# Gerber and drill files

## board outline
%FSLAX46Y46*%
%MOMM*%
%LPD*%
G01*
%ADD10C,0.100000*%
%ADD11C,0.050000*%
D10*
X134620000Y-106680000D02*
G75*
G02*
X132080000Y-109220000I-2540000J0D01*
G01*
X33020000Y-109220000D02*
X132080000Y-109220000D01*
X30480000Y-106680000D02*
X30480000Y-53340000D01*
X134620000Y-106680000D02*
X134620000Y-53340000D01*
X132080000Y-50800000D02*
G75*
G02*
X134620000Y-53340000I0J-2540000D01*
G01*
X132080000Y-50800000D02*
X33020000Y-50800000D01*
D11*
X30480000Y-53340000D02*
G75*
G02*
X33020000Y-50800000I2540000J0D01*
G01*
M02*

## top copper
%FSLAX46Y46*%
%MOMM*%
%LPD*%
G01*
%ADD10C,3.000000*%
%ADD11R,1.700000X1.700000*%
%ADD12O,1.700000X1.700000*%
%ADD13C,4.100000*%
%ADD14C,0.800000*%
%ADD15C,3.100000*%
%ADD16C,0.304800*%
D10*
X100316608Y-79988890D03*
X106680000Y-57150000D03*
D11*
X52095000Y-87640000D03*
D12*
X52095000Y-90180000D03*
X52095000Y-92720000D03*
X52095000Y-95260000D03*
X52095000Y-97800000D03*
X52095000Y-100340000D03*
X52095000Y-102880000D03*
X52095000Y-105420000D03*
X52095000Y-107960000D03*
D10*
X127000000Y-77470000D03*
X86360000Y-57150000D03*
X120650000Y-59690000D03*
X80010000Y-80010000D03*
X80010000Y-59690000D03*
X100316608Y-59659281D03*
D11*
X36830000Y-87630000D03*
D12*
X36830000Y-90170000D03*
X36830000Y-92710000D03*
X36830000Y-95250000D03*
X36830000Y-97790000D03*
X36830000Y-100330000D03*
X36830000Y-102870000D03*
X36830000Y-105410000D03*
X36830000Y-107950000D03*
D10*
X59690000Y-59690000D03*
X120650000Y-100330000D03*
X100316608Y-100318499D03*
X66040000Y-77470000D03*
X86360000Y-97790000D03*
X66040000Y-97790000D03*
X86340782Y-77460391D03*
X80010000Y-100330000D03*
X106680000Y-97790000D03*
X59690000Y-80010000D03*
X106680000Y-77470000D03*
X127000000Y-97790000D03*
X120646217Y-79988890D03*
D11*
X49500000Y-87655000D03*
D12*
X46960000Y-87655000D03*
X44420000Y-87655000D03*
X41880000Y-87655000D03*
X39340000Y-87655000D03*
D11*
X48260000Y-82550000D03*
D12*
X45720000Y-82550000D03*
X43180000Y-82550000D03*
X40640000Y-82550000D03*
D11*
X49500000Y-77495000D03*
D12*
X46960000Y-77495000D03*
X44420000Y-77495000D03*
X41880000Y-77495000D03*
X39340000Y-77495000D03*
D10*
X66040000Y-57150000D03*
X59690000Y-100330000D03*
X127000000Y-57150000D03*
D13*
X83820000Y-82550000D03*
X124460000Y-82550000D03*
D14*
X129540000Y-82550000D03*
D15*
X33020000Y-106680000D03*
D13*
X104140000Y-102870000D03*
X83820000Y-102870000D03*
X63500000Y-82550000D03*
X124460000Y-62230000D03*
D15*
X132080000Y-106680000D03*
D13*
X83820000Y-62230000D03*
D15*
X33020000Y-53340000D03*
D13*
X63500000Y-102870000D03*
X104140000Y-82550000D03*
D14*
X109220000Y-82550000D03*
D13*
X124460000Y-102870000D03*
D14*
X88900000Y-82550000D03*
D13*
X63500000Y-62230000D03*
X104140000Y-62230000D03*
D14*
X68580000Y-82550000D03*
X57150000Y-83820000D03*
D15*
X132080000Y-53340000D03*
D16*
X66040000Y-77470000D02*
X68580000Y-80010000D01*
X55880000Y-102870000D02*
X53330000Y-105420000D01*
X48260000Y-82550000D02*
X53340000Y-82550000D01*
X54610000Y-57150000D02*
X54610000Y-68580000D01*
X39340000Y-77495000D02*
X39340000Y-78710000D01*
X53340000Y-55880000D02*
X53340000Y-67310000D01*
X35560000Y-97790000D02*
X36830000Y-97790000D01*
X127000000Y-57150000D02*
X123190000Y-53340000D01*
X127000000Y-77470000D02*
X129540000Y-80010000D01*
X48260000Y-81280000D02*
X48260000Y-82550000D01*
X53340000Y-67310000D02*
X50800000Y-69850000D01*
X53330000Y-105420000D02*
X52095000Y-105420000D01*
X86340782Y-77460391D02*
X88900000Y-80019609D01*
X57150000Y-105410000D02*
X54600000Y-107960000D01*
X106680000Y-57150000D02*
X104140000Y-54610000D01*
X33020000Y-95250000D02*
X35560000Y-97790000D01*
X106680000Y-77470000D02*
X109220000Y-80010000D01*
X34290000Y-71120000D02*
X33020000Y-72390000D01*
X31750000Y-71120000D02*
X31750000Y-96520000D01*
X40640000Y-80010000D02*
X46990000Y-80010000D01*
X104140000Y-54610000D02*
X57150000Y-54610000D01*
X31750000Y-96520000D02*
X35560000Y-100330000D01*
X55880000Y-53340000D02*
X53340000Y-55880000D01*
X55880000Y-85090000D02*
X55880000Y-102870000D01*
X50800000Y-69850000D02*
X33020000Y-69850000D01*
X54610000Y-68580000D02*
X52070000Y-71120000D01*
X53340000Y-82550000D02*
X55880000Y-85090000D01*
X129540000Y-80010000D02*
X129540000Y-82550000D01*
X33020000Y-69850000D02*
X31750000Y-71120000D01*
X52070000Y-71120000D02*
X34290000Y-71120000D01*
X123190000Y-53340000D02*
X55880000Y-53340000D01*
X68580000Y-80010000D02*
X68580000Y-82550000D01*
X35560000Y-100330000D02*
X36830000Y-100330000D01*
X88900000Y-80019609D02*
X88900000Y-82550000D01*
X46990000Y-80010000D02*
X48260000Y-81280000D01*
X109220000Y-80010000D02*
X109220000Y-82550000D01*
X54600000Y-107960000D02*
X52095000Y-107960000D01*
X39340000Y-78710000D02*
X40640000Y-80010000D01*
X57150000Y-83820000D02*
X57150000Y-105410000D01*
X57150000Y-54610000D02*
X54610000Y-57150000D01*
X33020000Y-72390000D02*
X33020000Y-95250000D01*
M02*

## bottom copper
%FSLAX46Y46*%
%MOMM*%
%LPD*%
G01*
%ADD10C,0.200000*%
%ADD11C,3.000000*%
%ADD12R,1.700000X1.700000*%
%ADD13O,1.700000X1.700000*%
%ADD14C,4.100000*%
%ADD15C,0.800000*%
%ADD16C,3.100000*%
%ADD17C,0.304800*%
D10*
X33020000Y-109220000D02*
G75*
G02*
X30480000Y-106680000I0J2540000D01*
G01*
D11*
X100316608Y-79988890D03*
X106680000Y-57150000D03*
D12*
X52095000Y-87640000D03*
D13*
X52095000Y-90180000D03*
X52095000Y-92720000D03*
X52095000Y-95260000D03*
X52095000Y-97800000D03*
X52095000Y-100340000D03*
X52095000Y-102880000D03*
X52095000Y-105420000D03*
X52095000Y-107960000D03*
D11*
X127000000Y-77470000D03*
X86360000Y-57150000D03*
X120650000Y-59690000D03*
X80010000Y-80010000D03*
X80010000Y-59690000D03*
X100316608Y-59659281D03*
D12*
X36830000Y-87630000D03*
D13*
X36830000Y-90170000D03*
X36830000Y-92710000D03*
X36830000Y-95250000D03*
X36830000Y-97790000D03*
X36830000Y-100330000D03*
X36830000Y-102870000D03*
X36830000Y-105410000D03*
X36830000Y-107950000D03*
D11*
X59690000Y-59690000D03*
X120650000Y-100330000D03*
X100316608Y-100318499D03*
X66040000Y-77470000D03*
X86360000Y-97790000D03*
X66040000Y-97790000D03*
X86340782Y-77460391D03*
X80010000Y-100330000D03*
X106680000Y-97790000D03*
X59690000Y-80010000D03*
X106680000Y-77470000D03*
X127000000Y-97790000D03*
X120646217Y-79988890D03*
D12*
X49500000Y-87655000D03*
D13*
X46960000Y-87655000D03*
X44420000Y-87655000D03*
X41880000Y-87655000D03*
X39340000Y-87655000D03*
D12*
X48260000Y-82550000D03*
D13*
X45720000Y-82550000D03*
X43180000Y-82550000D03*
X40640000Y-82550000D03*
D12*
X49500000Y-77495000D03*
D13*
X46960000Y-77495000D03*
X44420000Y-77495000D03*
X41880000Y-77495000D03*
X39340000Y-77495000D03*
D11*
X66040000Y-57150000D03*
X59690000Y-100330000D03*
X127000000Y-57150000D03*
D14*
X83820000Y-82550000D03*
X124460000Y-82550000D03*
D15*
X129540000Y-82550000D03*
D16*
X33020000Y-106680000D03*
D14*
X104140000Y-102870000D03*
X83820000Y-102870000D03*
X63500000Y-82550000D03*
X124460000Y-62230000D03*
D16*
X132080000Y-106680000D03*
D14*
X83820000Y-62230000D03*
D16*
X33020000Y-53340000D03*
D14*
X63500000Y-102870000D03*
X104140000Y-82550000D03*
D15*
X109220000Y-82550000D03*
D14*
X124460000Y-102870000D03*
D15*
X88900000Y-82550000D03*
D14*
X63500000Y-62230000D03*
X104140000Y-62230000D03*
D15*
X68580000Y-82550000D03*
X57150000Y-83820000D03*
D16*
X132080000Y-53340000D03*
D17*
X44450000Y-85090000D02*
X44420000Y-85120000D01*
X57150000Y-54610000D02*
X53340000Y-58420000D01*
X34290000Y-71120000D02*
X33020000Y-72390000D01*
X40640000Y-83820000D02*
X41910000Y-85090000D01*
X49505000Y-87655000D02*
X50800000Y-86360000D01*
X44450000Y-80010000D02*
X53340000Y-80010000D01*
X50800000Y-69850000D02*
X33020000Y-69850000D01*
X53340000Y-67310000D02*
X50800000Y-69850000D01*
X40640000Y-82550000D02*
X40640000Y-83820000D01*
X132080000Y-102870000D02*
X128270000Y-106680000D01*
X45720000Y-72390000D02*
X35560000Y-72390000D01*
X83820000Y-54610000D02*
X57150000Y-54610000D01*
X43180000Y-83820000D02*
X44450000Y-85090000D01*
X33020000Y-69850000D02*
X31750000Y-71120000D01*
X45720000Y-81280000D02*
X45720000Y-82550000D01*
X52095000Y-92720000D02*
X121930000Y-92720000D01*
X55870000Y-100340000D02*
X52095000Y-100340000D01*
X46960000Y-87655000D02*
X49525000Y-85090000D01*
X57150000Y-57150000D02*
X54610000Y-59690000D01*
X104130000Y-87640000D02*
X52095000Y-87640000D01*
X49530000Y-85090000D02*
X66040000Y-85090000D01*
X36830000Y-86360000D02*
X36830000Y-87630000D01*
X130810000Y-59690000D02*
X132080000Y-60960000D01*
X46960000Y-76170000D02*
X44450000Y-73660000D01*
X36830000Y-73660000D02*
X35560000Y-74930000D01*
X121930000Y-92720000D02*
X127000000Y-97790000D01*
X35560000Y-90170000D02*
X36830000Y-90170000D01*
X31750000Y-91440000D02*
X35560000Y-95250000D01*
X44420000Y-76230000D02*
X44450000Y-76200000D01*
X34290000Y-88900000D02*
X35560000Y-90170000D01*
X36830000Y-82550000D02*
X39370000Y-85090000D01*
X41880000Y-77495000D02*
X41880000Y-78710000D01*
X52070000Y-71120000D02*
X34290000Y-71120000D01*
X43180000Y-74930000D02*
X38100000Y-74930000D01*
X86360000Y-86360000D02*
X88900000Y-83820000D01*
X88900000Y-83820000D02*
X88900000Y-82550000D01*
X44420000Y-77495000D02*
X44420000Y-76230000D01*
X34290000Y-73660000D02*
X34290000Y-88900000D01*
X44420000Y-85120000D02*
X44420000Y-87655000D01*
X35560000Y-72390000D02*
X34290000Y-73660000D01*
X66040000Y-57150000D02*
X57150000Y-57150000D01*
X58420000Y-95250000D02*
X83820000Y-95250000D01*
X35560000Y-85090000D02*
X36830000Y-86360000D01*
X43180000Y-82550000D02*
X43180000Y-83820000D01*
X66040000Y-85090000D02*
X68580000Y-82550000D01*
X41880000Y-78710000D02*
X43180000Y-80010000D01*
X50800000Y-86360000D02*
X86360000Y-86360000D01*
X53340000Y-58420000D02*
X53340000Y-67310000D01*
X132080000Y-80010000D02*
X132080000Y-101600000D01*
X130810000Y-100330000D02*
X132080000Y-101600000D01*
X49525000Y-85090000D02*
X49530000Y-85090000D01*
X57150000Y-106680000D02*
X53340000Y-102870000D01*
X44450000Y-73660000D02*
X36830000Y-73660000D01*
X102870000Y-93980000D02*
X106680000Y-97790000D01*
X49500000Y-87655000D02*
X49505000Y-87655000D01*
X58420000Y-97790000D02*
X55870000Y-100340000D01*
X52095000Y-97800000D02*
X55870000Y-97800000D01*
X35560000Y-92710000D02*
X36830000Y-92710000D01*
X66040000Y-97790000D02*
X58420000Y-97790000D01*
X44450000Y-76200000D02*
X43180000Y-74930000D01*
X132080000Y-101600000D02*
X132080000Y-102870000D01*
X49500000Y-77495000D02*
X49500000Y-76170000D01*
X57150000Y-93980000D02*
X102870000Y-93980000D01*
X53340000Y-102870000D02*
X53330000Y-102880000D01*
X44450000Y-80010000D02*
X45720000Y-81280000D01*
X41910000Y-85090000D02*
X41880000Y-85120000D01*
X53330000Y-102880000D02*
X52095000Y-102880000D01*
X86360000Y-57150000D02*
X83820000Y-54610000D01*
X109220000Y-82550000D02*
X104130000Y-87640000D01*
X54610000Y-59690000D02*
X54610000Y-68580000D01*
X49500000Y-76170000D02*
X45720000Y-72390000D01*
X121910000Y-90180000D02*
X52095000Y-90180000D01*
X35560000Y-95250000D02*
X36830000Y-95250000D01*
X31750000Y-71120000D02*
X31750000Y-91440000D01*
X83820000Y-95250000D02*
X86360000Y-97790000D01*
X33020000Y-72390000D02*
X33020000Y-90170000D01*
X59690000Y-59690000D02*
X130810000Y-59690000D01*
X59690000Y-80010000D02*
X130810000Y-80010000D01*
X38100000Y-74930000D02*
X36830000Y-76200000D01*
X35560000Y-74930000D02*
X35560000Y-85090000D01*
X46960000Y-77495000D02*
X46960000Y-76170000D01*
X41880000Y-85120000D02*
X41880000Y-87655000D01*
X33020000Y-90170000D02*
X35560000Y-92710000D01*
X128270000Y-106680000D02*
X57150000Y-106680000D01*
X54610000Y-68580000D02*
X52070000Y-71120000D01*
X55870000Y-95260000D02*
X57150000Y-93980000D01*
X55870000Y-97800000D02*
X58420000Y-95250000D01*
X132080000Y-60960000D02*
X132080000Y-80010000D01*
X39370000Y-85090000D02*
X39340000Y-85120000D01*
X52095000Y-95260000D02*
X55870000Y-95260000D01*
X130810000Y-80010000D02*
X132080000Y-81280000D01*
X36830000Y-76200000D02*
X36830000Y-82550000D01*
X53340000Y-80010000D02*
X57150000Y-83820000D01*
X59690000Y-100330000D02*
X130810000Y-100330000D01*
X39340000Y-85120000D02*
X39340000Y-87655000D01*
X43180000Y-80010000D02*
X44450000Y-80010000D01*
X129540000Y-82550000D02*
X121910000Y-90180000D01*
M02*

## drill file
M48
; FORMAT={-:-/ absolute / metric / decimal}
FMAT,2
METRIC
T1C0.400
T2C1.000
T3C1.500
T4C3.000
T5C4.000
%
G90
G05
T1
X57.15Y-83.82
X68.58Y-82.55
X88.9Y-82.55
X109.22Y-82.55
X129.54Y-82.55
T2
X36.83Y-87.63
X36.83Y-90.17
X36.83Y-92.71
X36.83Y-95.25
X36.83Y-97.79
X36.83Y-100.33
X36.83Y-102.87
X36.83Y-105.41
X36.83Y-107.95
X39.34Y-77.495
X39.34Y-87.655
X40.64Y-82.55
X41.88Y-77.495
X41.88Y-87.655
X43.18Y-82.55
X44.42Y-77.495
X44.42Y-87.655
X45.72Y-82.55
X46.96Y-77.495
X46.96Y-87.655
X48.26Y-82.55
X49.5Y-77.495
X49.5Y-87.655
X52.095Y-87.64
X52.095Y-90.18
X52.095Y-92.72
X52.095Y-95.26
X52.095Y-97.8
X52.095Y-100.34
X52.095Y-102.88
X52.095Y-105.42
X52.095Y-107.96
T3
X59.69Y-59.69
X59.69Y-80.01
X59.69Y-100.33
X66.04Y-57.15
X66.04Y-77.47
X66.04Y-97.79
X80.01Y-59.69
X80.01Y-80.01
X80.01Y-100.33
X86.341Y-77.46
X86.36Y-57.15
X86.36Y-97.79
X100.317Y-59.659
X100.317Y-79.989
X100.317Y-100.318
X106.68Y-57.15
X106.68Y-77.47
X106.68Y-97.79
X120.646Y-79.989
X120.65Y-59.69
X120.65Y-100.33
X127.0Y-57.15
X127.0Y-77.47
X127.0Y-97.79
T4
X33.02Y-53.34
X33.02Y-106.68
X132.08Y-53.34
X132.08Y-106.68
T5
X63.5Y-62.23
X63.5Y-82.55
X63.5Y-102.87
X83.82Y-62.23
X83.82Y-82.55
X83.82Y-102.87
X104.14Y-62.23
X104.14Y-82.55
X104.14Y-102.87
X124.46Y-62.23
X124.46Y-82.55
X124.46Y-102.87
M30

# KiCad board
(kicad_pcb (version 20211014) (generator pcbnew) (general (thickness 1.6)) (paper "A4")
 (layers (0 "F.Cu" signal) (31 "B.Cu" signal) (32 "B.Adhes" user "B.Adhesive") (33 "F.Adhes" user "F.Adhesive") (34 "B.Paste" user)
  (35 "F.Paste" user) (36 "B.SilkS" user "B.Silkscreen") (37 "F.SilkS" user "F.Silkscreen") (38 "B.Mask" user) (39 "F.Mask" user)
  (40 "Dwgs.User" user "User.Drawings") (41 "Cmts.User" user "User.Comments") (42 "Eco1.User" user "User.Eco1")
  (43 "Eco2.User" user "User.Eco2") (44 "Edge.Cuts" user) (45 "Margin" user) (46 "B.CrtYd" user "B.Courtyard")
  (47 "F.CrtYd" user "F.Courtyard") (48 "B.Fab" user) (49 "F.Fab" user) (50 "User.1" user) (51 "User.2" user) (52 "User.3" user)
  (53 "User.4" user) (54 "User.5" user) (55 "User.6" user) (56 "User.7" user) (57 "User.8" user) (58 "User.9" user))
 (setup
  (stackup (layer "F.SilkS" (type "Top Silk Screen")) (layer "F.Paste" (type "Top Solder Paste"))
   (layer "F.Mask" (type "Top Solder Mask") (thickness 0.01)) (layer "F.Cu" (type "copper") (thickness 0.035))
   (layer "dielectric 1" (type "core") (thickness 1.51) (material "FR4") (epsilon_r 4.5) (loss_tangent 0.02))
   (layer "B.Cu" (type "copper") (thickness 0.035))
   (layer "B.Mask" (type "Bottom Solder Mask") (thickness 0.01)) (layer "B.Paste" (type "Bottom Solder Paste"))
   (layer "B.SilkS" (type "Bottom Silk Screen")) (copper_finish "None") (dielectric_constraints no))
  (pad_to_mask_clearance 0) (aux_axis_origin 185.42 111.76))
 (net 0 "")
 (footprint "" (layer "F.Cu") (at 100.316608 79.98889)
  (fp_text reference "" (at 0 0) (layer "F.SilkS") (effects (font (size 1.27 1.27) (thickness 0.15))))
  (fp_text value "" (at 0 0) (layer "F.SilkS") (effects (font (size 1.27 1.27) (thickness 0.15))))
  (pad "1" thru_hole circle (at 0 0) (size 3 3) (drill 1.5) (layers *.Cu *.Mask)))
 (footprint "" (layer "F.Cu") (at 106.68 57.15)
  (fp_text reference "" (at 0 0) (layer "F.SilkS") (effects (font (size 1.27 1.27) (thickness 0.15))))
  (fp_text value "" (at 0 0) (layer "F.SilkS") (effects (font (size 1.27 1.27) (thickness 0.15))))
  (pad "1" thru_hole circle (at 0 0) (size 3 3) (drill 1.5) (layers *.Cu *.Mask)))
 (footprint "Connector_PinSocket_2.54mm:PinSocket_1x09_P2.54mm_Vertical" (layer "F.Cu") (at 52.095 87.64)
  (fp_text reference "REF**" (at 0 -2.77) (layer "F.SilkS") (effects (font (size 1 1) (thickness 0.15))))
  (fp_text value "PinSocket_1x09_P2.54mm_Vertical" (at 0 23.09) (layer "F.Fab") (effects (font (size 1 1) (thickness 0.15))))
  (pad "1" thru_hole rect (at 0 0) (size 1.7 1.7) (drill 1) (layers *.Cu *.Mask))
  (pad "2" thru_hole oval (at 0 2.54) (size 1.7 1.7) (drill 1) (layers *.Cu *.Mask))
  (pad "3" thru_hole oval (at 0 5.08) (size 1.7 1.7) (drill 1) (layers *.Cu *.Mask))
  (pad "4" thru_hole oval (at 0 7.62) (size 1.7 1.7) (drill 1) (layers *.Cu *.Mask))
  (pad "5" thru_hole oval (at 0 10.16) (size 1.7 1.7) (drill 1) (layers *.Cu *.Mask))
  (pad "6" thru_hole oval (at 0 12.7) (size 1.7 1.7) (drill 1) (layers *.Cu *.Mask))
  (pad "7" thru_hole oval (at 0 15.24) (size 1.7 1.7) (drill 1) (layers *.Cu *.Mask))
  (pad "8" thru_hole oval (at 0 17.78) (size 1.7 1.7) (drill 1) (layers *.Cu *.Mask))
  (pad "9" thru_hole oval (at 0 20.32) (size 1.7 1.7) (drill 1) (layers *.Cu *.Mask)))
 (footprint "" (layer "F.Cu") (at 127 77.47)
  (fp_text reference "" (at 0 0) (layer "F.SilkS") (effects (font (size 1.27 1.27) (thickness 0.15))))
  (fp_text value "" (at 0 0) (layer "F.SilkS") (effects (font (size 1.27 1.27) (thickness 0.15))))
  (pad "1" thru_hole circle (at 0 0) (size 3 3) (drill 1.5) (layers *.Cu *.Mask)))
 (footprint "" (layer "F.Cu") (at 86.36 57.15)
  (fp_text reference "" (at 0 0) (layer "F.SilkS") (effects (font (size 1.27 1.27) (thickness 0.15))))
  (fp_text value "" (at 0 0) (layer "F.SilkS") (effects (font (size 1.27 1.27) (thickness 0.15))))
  (pad "1" thru_hole circle (at 0 0) (size 3 3) (drill 1.5) (layers *.Cu *.Mask)))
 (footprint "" (layer "F.Cu") (at 120.65 59.69)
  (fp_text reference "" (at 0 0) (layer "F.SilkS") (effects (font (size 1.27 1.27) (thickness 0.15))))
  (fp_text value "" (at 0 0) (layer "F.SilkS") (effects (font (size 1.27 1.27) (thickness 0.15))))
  (pad "1" thru_hole circle (at 0 0) (size 3 3) (drill 1.5) (layers *.Cu *.Mask)))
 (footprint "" (layer "F.Cu") (at 80.01 80.01)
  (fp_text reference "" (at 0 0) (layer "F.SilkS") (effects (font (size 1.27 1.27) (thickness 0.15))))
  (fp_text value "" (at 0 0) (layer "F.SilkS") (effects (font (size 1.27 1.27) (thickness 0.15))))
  (pad "1" thru_hole circle (at 0 0) (size 3 3) (drill 1.5) (layers *.Cu *.Mask)))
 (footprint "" (layer "F.Cu") (at 80.01 59.69)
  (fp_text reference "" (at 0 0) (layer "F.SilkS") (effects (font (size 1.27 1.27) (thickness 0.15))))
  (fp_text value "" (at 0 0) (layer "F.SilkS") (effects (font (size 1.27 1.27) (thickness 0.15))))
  (pad "1" thru_hole circle (at 0 0) (size 3 3) (drill 1.5) (layers *.Cu *.Mask)))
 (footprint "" (layer "F.Cu") (at 100.316608 59.659281)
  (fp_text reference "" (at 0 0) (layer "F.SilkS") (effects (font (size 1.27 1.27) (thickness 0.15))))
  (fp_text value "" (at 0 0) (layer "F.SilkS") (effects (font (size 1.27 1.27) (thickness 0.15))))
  (pad "1" thru_hole circle (at 0 0) (size 3 3) (drill 1.5) (layers *.Cu *.Mask)))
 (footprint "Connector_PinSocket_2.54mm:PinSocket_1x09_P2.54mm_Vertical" (layer "F.Cu") (at 36.83 87.63)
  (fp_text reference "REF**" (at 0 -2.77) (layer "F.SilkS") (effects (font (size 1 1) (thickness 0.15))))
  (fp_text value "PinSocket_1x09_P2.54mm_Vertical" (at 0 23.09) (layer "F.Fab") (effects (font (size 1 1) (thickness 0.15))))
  (pad "1" thru_hole rect (at 0 0) (size 1.7 1.7) (drill 1) (layers *.Cu *.Mask))
  (pad "2" thru_hole oval (at 0 2.54) (size 1.7 1.7) (drill 1) (layers *.Cu *.Mask))
  (pad "3" thru_hole oval (at 0 5.08) (size 1.7 1.7) (drill 1) (layers *.Cu *.Mask))
  (pad "4" thru_hole oval (at 0 7.62) (size 1.7 1.7) (drill 1) (layers *.Cu *.Mask))
  (pad "5" thru_hole oval (at 0 10.16) (size 1.7 1.7) (drill 1) (layers *.Cu *.Mask))
  (pad "6" thru_hole oval (at 0 12.7) (size 1.7 1.7) (drill 1) (layers *.Cu *.Mask))
  (pad "7" thru_hole oval (at 0 15.24) (size 1.7 1.7) (drill 1) (layers *.Cu *.Mask))
  (pad "8" thru_hole oval (at 0 17.78) (size 1.7 1.7) (drill 1) (layers *.Cu *.Mask))
  (pad "9" thru_hole oval (at 0 20.32) (size 1.7 1.7) (drill 1) (layers *.Cu *.Mask)))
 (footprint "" (layer "F.Cu") (at 59.69 59.69)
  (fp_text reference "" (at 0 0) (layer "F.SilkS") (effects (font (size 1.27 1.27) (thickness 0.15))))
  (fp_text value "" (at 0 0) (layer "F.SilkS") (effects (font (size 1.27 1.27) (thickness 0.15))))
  (pad "1" thru_hole circle (at 0 0) (size 3 3) (drill 1.5) (layers *.Cu *.Mask)))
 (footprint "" (layer "F.Cu") (at 120.65 100.33)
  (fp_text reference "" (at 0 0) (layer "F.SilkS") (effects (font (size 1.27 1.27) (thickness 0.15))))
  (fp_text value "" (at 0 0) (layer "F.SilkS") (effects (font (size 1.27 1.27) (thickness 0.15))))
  (pad "1" thru_hole circle (at 0 0) (size 3 3) (drill 1.5) (layers *.Cu *.Mask)))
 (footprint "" (layer "F.Cu") (at 100.316608 100.318499)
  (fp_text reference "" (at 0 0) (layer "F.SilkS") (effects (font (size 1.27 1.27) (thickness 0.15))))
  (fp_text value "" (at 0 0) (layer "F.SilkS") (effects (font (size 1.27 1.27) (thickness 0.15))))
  (pad "1" thru_hole circle (at 0 0) (size 3 3) (drill 1.5) (layers *.Cu *.Mask)))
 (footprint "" (layer "F.Cu") (at 66.04 77.47)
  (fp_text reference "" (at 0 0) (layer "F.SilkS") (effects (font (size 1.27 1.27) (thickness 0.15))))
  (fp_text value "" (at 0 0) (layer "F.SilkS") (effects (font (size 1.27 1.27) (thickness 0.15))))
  (pad "1" thru_hole circle (at 0 0) (size 3 3) (drill 1.5) (layers *.Cu *.Mask)))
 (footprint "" (layer "F.Cu") (at 86.36 97.79)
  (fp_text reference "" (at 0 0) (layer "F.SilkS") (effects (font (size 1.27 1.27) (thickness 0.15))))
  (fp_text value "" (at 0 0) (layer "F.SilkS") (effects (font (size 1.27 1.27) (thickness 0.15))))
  (pad "1" thru_hole circle (at 0 0) (size 3 3) (drill 1.5) (layers *.Cu *.Mask)))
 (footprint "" (layer "F.Cu") (at 66.04 97.79)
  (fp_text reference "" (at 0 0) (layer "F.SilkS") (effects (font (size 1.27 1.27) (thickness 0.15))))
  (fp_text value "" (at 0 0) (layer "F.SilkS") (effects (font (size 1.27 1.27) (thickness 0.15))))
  (pad "1" thru_hole circle (at 0 0) (size 3 3) (drill 1.5) (layers *.Cu *.Mask)))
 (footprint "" (layer "F.Cu") (at 86.340782 77.460391)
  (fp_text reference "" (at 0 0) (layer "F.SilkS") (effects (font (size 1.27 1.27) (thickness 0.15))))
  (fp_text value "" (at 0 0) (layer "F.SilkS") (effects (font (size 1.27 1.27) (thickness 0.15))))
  (pad "1" thru_hole circle (at 0 0) (size 3 3) (drill 1.5) (layers *.Cu *.Mask)))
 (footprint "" (layer "F.Cu") (at 80.01 100.33)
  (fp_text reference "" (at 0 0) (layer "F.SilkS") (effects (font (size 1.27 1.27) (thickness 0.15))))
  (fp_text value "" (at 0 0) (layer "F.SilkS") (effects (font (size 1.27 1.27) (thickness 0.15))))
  (pad "1" thru_hole circle (at 0 0) (size 3 3) (drill 1.5) (layers *.Cu *.Mask)))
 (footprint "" (layer "F.Cu") (at 106.68 97.79)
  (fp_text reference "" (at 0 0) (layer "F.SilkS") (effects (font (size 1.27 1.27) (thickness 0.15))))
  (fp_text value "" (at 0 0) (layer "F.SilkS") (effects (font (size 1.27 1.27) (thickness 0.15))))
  (pad "1" thru_hole circle (at 0 0) (size 3 3) (drill 1.5) (layers *.Cu *.Mask)))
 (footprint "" (layer "F.Cu") (at 59.69 80.01)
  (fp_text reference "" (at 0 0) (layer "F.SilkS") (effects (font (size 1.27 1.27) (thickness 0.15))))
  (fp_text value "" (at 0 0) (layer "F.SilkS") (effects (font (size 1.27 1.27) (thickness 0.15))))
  (pad "1" thru_hole circle (at 0 0) (size 3 3) (drill 1.5) (layers *.Cu *.Mask)))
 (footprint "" (layer "F.Cu") (at 106.68 77.47)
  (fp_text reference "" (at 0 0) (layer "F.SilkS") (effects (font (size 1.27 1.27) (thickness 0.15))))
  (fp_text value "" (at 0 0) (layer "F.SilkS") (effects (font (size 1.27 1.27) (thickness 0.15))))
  (pad "1" thru_hole circle (at 0 0) (size 3 3) (drill 1.5) (layers *.Cu *.Mask)))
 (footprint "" (layer "F.Cu") (at 127 97.79)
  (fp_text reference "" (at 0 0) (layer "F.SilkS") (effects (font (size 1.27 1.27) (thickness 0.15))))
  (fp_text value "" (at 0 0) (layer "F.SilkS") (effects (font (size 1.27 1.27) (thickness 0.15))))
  (pad "1" thru_hole circle (at 0 0) (size 3 3) (drill 1.5) (layers *.Cu *.Mask)))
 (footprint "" (layer "F.Cu") (at 120.646217 79.98889)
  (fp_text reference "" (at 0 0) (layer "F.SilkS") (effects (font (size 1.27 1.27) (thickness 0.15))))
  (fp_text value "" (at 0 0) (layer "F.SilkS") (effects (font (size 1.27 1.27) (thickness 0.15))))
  (pad "1" thru_hole circle (at 0 0) (size 3 3) (drill 1.5) (layers *.Cu *.Mask)))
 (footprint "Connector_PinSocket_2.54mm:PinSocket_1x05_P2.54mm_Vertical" (layer "F.Cu") (at 49.5 87.655 -90)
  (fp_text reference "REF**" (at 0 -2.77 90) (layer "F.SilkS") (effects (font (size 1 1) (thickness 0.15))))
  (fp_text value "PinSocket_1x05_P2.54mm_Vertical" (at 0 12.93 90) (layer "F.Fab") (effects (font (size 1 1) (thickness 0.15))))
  (pad "1" thru_hole rect (at 0 0 270) (size 1.7 1.7) (drill 1) (layers *.Cu *.Mask))
  (pad "2" thru_hole oval (at 0 2.54 270) (size 1.7 1.7) (drill 1) (layers *.Cu *.Mask))
  (pad "3" thru_hole oval (at 0 5.08 270) (size 1.7 1.7) (drill 1) (layers *.Cu *.Mask))
  (pad "4" thru_hole oval (at 0 7.62 270) (size 1.7 1.7) (drill 1) (layers *.Cu *.Mask))
  (pad "5" thru_hole oval (at 0 10.16 270) (size 1.7 1.7) (drill 1) (layers *.Cu *.Mask)))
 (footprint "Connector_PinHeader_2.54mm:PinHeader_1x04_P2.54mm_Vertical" (layer "F.Cu") (at 48.26 82.55 -90)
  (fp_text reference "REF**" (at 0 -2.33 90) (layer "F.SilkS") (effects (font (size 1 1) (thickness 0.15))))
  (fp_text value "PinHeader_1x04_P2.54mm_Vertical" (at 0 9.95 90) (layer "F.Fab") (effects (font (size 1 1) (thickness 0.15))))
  (pad "1" thru_hole rect (at 0 0 270) (size 1.7 1.7) (drill 1) (layers *.Cu *.Mask))
  (pad "2" thru_hole oval (at 0 2.54 270) (size 1.7 1.7) (drill 1) (layers *.Cu *.Mask))
  (pad "3" thru_hole oval (at 0 5.08 270) (size 1.7 1.7) (drill 1) (layers *.Cu *.Mask))
  (pad "4" thru_hole oval (at 0 7.62 270) (size 1.7 1.7) (drill 1) (layers *.Cu *.Mask)))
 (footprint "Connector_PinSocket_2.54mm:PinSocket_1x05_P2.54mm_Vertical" (layer "F.Cu") (at 49.5 77.495 -90)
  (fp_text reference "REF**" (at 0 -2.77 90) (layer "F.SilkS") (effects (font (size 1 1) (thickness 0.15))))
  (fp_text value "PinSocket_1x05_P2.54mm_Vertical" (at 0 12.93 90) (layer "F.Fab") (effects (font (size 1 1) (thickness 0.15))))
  (pad "1" thru_hole rect (at 0 0 270) (size 1.7 1.7) (drill 1) (layers *.Cu *.Mask))
  (pad "2" thru_hole oval (at 0 2.54 270) (size 1.7 1.7) (drill 1) (layers *.Cu *.Mask))
  (pad "3" thru_hole oval (at 0 5.08 270) (size 1.7 1.7) (drill 1) (layers *.Cu *.Mask))
  (pad "4" thru_hole oval (at 0 7.62 270) (size 1.7 1.7) (drill 1) (layers *.Cu *.Mask))
  (pad "5" thru_hole oval (at 0 10.16 270) (size 1.7 1.7) (drill 1) (layers *.Cu *.Mask)))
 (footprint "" (layer "F.Cu") (at 66.04 57.15)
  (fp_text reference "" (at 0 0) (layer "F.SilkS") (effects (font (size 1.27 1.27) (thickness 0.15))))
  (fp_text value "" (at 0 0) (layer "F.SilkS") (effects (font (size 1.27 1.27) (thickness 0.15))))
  (pad "1" thru_hole circle (at 0 0) (size 3 3) (drill 1.5) (layers *.Cu *.Mask)))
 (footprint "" (layer "F.Cu") (at 59.69 100.33)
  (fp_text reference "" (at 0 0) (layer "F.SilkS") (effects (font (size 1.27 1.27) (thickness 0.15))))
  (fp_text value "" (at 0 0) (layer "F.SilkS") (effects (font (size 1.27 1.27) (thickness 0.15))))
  (pad "1" thru_hole circle (at 0 0) (size 3 3) (drill 1.5) (layers *.Cu *.Mask)))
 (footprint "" (layer "F.Cu") (at 127 57.15)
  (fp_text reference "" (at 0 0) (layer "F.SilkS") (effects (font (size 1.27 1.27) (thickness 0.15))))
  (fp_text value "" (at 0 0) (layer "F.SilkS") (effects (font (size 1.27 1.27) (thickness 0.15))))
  (pad "1" thru_hole circle (at 0 0) (size 3 3) (drill 1.5) (layers *.Cu *.Mask)))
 (gr_arc (start 33.02 109.22) (mid 31.223949 108.476051) (end 30.48 106.68) (layer "B.Cu") (width 0.2))
 (gr_arc (start 134.62 106.68) (mid 133.876051 108.476051) (end 132.08 109.22) (layer "Edge.Cuts") (width 0.1))
 (gr_line (start 33.02 109.22) (end 132.08 109.22) (layer "Edge.Cuts") (width 0.1))
 (gr_line (start 30.48 106.68) (end 30.48 53.34) (layer "Edge.Cuts") (width 0.1))
 (gr_line (start 134.62 106.68) (end 134.62 53.34) (layer "Edge.Cuts") (width 0.1))
 (gr_arc (start 132.08 50.8) (mid 133.876051 51.543949) (end 134.62 53.34) (layer "Edge.Cuts") (width 0.1))
 (gr_line (start 132.08 50.8) (end 33.02 50.8) (layer "Edge.Cuts") (width 0.1))
 (gr_arc (start 30.48 53.34) (mid 31.223949 51.543949) (end 33.02 50.8) (layer "Edge.Cuts") (width 0.05))
 (segment (start 66.04 77.47) (end 68.58 80.01) (width 0.3048) (layer "F.Cu") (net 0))
 (segment (start 55.88 102.87) (end 53.33 105.42) (width 0.3048) (layer "F.Cu") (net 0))
 (segment (start 48.26 82.55) (end 53.34 82.55) (width 0.3048) (layer "F.Cu") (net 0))
 (segment (start 54.61 57.15) (end 54.61 68.58) (width 0.3048) (layer "F.Cu") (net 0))
 (segment (start 39.34 77.495) (end 39.34 78.71) (width 0.3048) (layer "F.Cu") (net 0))
 (segment (start 53.34 55.88) (end 53.34 67.31) (width 0.3048) (layer "F.Cu") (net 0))
 (segment (start 35.56 97.79) (end 36.83 97.79) (width 0.3048) (layer "F.Cu") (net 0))
 (segment (start 127 57.15) (end 123.19 53.34) (width 0.3048) (layer "F.Cu") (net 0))
 (segment (start 127 77.47) (end 129.54 80.01) (width 0.3048) (layer "F.Cu") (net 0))
 (segment (start 48.26 81.28) (end 48.26 82.55) (width 0.3048) (layer "F.Cu") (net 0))
 (segment (start 53.34 67.31) (end 50.8 69.85) (width 0.3048) (layer "F.Cu") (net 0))
 (segment (start 53.33 105.42) (end 52.095 105.42) (width 0.3048) (layer "F.Cu") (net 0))
 (segment (start 86.340782 77.460391) (end 88.9 80.019609) (width 0.3048) (layer "F.Cu") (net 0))
 (segment (start 57.15 105.41) (end 54.6 107.96) (width 0.3048) (layer "F.Cu") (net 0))
 (segment (start 106.68 57.15) (end 104.14 54.61) (width 0.3048) (layer "F.Cu") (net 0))
 (segment (start 33.02 95.25) (end 35.56 97.79) (width 0.3048) (layer "F.Cu") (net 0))
 (segment (start 106.68 77.47) (end 109.22 80.01) (width 0.3048) (layer "F.Cu") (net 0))
 (segment (start 34.29 71.12) (end 33.02 72.39) (width 0.3048) (layer "F.Cu") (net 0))
 (segment (start 31.75 71.12) (end 31.75 96.52) (width 0.3048) (layer "F.Cu") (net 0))
 (segment (start 40.64 80.01) (end 46.99 80.01) (width 0.3048) (layer "F.Cu") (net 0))
 (segment (start 104.14 54.61) (end 57.15 54.61) (width 0.3048) (layer "F.Cu") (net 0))
 (segment (start 31.75 96.52) (end 35.56 100.33) (width 0.3048) (layer "F.Cu") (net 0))
 (segment (start 55.88 53.34) (end 53.34 55.88) (width 0.3048) (layer "F.Cu") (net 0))
 (segment (start 55.88 85.09) (end 55.88 102.87) (width 0.3048) (layer "F.Cu") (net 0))
 (segment (start 50.8 69.85) (end 33.02 69.85) (width 0.3048) (layer "F.Cu") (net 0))
 (segment (start 54.61 68.58) (end 52.07 71.12) (width 0.3048) (layer "F.Cu") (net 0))
 (segment (start 53.34 82.55) (end 55.88 85.09) (width 0.3048) (layer "F.Cu") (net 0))
 (segment (start 129.54 80.01) (end 129.54 82.55) (width 0.3048) (layer "F.Cu") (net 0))
 (segment (start 33.02 69.85) (end 31.75 71.12) (width 0.3048) (layer "F.Cu") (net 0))
 (segment (start 52.07 71.12) (end 34.29 71.12) (width 0.3048) (layer "F.Cu") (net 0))
 (segment (start 123.19 53.34) (end 55.88 53.34) (width 0.3048) (layer "F.Cu") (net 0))
 (segment (start 68.58 80.01) (end 68.58 82.55) (width 0.3048) (layer "F.Cu") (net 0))
 (segment (start 35.56 100.33) (end 36.83 100.33) (width 0.3048) (layer "F.Cu") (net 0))
 (segment (start 88.9 80.019609) (end 88.9 82.55) (width 0.3048) (layer "F.Cu") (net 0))
 (segment (start 46.99 80.01) (end 48.26 81.28) (width 0.3048) (layer "F.Cu") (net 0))
 (segment (start 109.22 80.01) (end 109.22 82.55) (width 0.3048) (layer "F.Cu") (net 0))
 (segment (start 54.6 107.96) (end 52.095 107.96) (width 0.3048) (layer "F.Cu") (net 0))
 (segment (start 39.34 78.71) (end 40.64 80.01) (width 0.3048) (layer "F.Cu") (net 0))
 (segment (start 57.15 83.82) (end 57.15 105.41) (width 0.3048) (layer "F.Cu") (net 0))
 (segment (start 57.15 54.61) (end 54.61 57.15) (width 0.3048) (layer "F.Cu") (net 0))
 (segment (start 33.02 72.39) (end 33.02 95.25) (width 0.3048) (layer "F.Cu") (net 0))
 (via (at 83.82 82.55) (size 4.1) (drill 4) (layers "F.Cu" "B.Cu") (free) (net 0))
 (via (at 124.46 82.55) (size 4.1) (drill 4) (layers "F.Cu" "B.Cu") (free) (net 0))
 (via (at 129.54 82.55) (size 0.8) (drill 0.4) (layers "F.Cu" "B.Cu") (free) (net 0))
 (via (at 33.02 106.68) (size 3.1) (drill 3) (layers "F.Cu" "B.Cu") (free) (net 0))
 (via (at 104.14 102.87) (size 4.1) (drill 4) (layers "F.Cu" "B.Cu") (free) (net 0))
 (via (at 83.82 102.87) (size 4.1) (drill 4) (layers "F.Cu" "B.Cu") (free) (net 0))
 (via (at 63.5 82.55) (size 4.1) (drill 4) (layers "F.Cu" "B.Cu") (free) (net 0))
 (via (at 124.46 62.23) (size 4.1) (drill 4) (layers "F.Cu" "B.Cu") (free) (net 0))
 (via (at 132.08 106.68) (size 3.1) (drill 3) (layers "F.Cu" "B.Cu") (free) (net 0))
 (via (at 83.82 62.23) (size 4.1) (drill 4) (layers "F.Cu" "B.Cu") (free) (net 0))
 (via (at 33.02 53.34) (size 3.1) (drill 3) (layers "F.Cu" "B.Cu") (free) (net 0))
 (via (at 63.5 102.87) (size 4.1) (drill 4) (layers "F.Cu" "B.Cu") (free) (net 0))
 (via (at 104.14 82.55) (size 4.1) (drill 4) (layers "F.Cu" "B.Cu") (free) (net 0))
 (via (at 109.22 82.55) (size 0.8) (drill 0.4) (layers "F.Cu" "B.Cu") (free) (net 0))
 (via (at 124.46 102.87) (size 4.1) (drill 4) (layers "F.Cu" "B.Cu") (free) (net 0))
 (via (at 88.9 82.55) (size 0.8) (drill 0.4) (layers "F.Cu" "B.Cu") (free) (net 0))
 (via (at 63.5 62.23) (size 4.1) (drill 4) (layers "F.Cu" "B.Cu") (free) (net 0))
 (via (at 104.14 62.23) (size 4.1) (drill 4) (layers "F.Cu" "B.Cu") (free) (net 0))
 (via (at 68.58 82.55) (size 0.8) (drill 0.4) (layers "F.Cu" "B.Cu") (free) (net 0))
 (via (at 57.15 83.82) (size 0.8) (drill 0.4) (layers "F.Cu" "B.Cu") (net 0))
 (via (at 132.08 53.34) (size 3.1) (drill 3) (layers "F.Cu" "B.Cu") (free) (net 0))
 (segment (start 44.45 85.09) (end 44.42 85.12) (width 0.3048) (layer "B.Cu") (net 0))
 (segment (start 57.15 54.61) (end 53.34 58.42) (width 0.3048) (layer "B.Cu") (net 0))
 (segment (start 34.29 71.12) (end 33.02 72.39) (width 0.3048) (layer "B.Cu") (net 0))
 (segment (start 40.64 83.82) (end 41.91 85.09) (width 0.3048) (layer "B.Cu") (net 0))
 (segment (start 49.505 87.655) (end 50.8 86.36) (width 0.3048) (layer "B.Cu") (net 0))
 (segment (start 44.45 80.01) (end 53.34 80.01) (width 0.3048) (layer "B.Cu") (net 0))
 (segment (start 50.8 69.85) (end 33.02 69.85) (width 0.3048) (layer "B.Cu") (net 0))
 (segment (start 53.34 67.31) (end 50.8 69.85) (width 0.3048) (layer "B.Cu") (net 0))
 (segment (start 40.64 82.55) (end 40.64 83.82) (width 0.3048) (layer "B.Cu") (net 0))
 (segment (start 132.08 102.87) (end 128.27 106.68) (width 0.3048) (layer "B.Cu") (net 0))
 (segment (start 45.72 72.39) (end 35.56 72.39) (width 0.3048) (layer "B.Cu") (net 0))
 (segment (start 83.82 54.61) (end 57.15 54.61) (width 0.3048) (layer "B.Cu") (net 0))
 (segment (start 43.18 83.82) (end 44.45 85.09) (width 0.3048) (layer "B.Cu") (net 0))
 (segment (start 33.02 69.85) (end 31.75 71.12) (width 0.3048) (layer "B.Cu") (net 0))
 (segment (start 45.72 81.28) (end 45.72 82.55) (width 0.3048) (layer "B.Cu") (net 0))
 (segment (start 52.095 92.72) (end 121.93 92.72) (width 0.3048) (layer "B.Cu") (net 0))
 (segment (start 55.87 100.34) (end 52.095 100.34) (width 0.3048) (layer "B.Cu") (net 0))
 (segment (start 46.96 87.655) (end 49.525 85.09) (width 0.3048) (layer "B.Cu") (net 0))
 (segment (start 57.15 57.15) (end 54.61 59.69) (width 0.3048) (layer "B.Cu") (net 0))
 (segment (start 104.13 87.64) (end 52.095 87.64) (width 0.3048) (layer "B.Cu") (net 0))
 (segment (start 49.53 85.09) (end 66.04 85.09) (width 0.3048) (layer "B.Cu") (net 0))
 (segment (start 36.83 86.36) (end 36.83 87.63) (width 0.3048) (layer "B.Cu") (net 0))
 (segment (start 130.81 59.69) (end 132.08 60.96) (width 0.3048) (layer "B.Cu") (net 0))
 (segment (start 46.96 76.17) (end 44.45 73.66) (width 0.3048) (layer "B.Cu") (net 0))
 (segment (start 36.83 73.66) (end 35.56 74.93) (width 0.3048) (layer "B.Cu") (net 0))
 (segment (start 121.93 92.72) (end 127 97.79) (width 0.3048) (layer "B.Cu") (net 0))
 (segment (start 35.56 90.17) (end 36.83 90.17) (width 0.3048) (layer "B.Cu") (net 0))
 (segment (start 31.75 91.44) (end 35.56 95.25) (width 0.3048) (layer "B.Cu") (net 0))
 (segment (start 44.42 76.23) (end 44.45 76.2) (width 0.3048) (layer "B.Cu") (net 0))
 (segment (start 34.29 88.9) (end 35.56 90.17) (width 0.3048) (layer "B.Cu") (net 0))
 (segment (start 36.83 82.55) (end 39.37 85.09) (width 0.3048) (layer "B.Cu") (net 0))
 (segment (start 41.88 77.495) (end 41.88 78.71) (width 0.3048) (layer "B.Cu") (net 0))
 (segment (start 52.07 71.12) (end 34.29 71.12) (width 0.3048) (layer "B.Cu") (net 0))
 (segment (start 43.18 74.93) (end 38.1 74.93) (width 0.3048) (layer "B.Cu") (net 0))
 (segment (start 86.36 86.36) (end 88.9 83.82) (width 0.3048) (layer "B.Cu") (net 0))
 (segment (start 88.9 83.82) (end 88.9 82.55) (width 0.3048) (layer "B.Cu") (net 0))
 (segment (start 44.42 77.495) (end 44.42 76.23) (width 0.3048) (layer "B.Cu") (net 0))
 (segment (start 34.29 73.66) (end 34.29 88.9) (width 0.3048) (layer "B.Cu") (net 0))
 (segment (start 44.42 85.12) (end 44.42 87.655) (width 0.3048) (layer "B.Cu") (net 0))
 (segment (start 35.56 72.39) (end 34.29 73.66) (width 0.3048) (layer "B.Cu") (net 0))
 (segment (start 66.04 57.15) (end 57.15 57.15) (width 0.3048) (layer "B.Cu") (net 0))
 (segment (start 58.42 95.25) (end 83.82 95.25) (width 0.3048) (layer "B.Cu") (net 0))
 (segment (start 35.56 85.09) (end 36.83 86.36) (width 0.3048) (layer "B.Cu") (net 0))
 (segment (start 43.18 82.55) (end 43.18 83.82) (width 0.3048) (layer "B.Cu") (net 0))
 (segment (start 66.04 85.09) (end 68.58 82.55) (width 0.3048) (layer "B.Cu") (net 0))
 (segment (start 41.88 78.71) (end 43.18 80.01) (width 0.3048) (layer "B.Cu") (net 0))
 (segment (start 50.8 86.36) (end 86.36 86.36) (width 0.3048) (layer "B.Cu") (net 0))
 (segment (start 53.34 58.42) (end 53.34 67.31) (width 0.3048) (layer "B.Cu") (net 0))
 (segment (start 132.08 80.01) (end 132.08 101.6) (width 0.3048) (layer "B.Cu") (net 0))
 (segment (start 130.81 100.33) (end 132.08 101.6) (width 0.3048) (layer "B.Cu") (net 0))
 (segment (start 49.525 85.09) (end 49.53 85.09) (width 0.3048) (layer "B.Cu") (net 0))
 (segment (start 57.15 106.68) (end 53.34 102.87) (width 0.3048) (layer "B.Cu") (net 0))
 (segment (start 44.45 73.66) (end 36.83 73.66) (width 0.3048) (layer "B.Cu") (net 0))
 (segment (start 102.87 93.98) (end 106.68 97.79) (width 0.3048) (layer "B.Cu") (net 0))
 (segment (start 49.5 87.655) (end 49.505 87.655) (width 0.3048) (layer "B.Cu") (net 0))
 (segment (start 58.42 97.79) (end 55.87 100.34) (width 0.3048) (layer "B.Cu") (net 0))
 (segment (start 52.095 97.8) (end 55.87 97.8) (width 0.3048) (layer "B.Cu") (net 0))
 (segment (start 35.56 92.71) (end 36.83 92.71) (width 0.3048) (layer "B.Cu") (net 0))
 (segment (start 66.04 97.79) (end 58.42 97.79) (width 0.3048) (layer "B.Cu") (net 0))
 (segment (start 44.45 76.2) (end 43.18 74.93) (width 0.3048) (layer "B.Cu") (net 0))
 (segment (start 132.08 101.6) (end 132.08 102.87) (width 0.3048) (layer "B.Cu") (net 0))
 (segment (start 49.5 77.495) (end 49.5 76.17) (width 0.3048) (layer "B.Cu") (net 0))
 (segment (start 57.15 93.98) (end 102.87 93.98) (width 0.3048) (layer "B.Cu") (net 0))
 (segment (start 53.34 102.87) (end 53.33 102.88) (width 0.3048) (layer "B.Cu") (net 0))
 (segment (start 44.45 80.01) (end 45.72 81.28) (width 0.3048) (layer "B.Cu") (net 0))
 (segment (start 41.91 85.09) (end 41.88 85.12) (width 0.3048) (layer "B.Cu") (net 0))
 (segment (start 53.33 102.88) (end 52.095 102.88) (width 0.3048) (layer "B.Cu") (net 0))
 (segment (start 86.36 57.15) (end 83.82 54.61) (width 0.3048) (layer "B.Cu") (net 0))
 (segment (start 109.22 82.55) (end 104.13 87.64) (width 0.3048) (layer "B.Cu") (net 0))
 (segment (start 54.61 59.69) (end 54.61 68.58) (width 0.3048) (layer "B.Cu") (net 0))
 (segment (start 49.5 76.17) (end 45.72 72.39) (width 0.3048) (layer "B.Cu") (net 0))
 (segment (start 121.91 90.18) (end 52.095 90.18) (width 0.3048) (layer "B.Cu") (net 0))
 (segment (start 35.56 95.25) (end 36.83 95.25) (width 0.3048) (layer "B.Cu") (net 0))
 (segment (start 31.75 71.12) (end 31.75 91.44) (width 0.3048) (layer "B.Cu") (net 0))
 (segment (start 83.82 95.25) (end 86.36 97.79) (width 0.3048) (layer "B.Cu") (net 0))
 (segment (start 33.02 72.39) (end 33.02 90.17) (width 0.3048) (layer "B.Cu") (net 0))
 (segment (start 59.69 59.69) (end 130.81 59.69) (width 0.3048) (layer "B.Cu") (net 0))
 (segment (start 59.69 80.01) (end 130.81 80.01) (width 0.3048) (layer "B.Cu") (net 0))
 (segment (start 38.1 74.93) (end 36.83 76.2) (width 0.3048) (layer "B.Cu") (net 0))
 (segment (start 35.56 74.93) (end 35.56 85.09) (width 0.3048) (layer "B.Cu") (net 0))
 (segment (start 46.96 77.495) (end 46.96 76.17) (width 0.3048) (layer "B.Cu") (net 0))
 (segment (start 41.88 85.12) (end 41.88 87.655) (width 0.3048) (layer "B.Cu") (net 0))
 (segment (start 33.02 90.17) (end 35.56 92.71) (width 0.3048) (layer "B.Cu") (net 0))
 (segment (start 128.27 106.68) (end 57.15 106.68) (width 0.3048) (layer "B.Cu") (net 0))
 (segment (start 54.61 68.58) (end 52.07 71.12) (width 0.3048) (layer "B.Cu") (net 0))
 (segment (start 55.87 95.26) (end 57.15 93.98) (width 0.3048) (layer "B.Cu") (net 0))
 (segment (start 55.87 97.8) (end 58.42 95.25) (width 0.3048) (layer "B.Cu") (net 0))
 (segment (start 132.08 60.96) (end 132.08 80.01) (width 0.3048) (layer "B.Cu") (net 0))
 (segment (start 39.37 85.09) (end 39.34 85.12) (width 0.3048) (layer "B.Cu") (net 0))
 (segment (start 52.095 95.26) (end 55.87 95.26) (width 0.3048) (layer "B.Cu") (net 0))
 (segment (start 130.81 80.01) (end 132.08 81.28) (width 0.3048) (layer "B.Cu") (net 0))
 (segment (start 36.83 76.2) (end 36.83 82.55) (width 0.3048) (layer "B.Cu") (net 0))
 (segment (start 53.34 80.01) (end 57.15 83.82) (width 0.3048) (layer "B.Cu") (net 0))
 (segment (start 59.69 100.33) (end 130.81 100.33) (width 0.3048) (layer "B.Cu") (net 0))
 (segment (start 39.34 85.12) (end 39.34 87.655) (width 0.3048) (layer "B.Cu") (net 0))
 (segment (start 43.18 80.01) (end 44.45 80.01) (width 0.3048) (layer "B.Cu") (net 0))
 (segment (start 129.54 82.55) (end 121.91 90.18) (width 0.3048) (layer "B.Cu") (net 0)))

